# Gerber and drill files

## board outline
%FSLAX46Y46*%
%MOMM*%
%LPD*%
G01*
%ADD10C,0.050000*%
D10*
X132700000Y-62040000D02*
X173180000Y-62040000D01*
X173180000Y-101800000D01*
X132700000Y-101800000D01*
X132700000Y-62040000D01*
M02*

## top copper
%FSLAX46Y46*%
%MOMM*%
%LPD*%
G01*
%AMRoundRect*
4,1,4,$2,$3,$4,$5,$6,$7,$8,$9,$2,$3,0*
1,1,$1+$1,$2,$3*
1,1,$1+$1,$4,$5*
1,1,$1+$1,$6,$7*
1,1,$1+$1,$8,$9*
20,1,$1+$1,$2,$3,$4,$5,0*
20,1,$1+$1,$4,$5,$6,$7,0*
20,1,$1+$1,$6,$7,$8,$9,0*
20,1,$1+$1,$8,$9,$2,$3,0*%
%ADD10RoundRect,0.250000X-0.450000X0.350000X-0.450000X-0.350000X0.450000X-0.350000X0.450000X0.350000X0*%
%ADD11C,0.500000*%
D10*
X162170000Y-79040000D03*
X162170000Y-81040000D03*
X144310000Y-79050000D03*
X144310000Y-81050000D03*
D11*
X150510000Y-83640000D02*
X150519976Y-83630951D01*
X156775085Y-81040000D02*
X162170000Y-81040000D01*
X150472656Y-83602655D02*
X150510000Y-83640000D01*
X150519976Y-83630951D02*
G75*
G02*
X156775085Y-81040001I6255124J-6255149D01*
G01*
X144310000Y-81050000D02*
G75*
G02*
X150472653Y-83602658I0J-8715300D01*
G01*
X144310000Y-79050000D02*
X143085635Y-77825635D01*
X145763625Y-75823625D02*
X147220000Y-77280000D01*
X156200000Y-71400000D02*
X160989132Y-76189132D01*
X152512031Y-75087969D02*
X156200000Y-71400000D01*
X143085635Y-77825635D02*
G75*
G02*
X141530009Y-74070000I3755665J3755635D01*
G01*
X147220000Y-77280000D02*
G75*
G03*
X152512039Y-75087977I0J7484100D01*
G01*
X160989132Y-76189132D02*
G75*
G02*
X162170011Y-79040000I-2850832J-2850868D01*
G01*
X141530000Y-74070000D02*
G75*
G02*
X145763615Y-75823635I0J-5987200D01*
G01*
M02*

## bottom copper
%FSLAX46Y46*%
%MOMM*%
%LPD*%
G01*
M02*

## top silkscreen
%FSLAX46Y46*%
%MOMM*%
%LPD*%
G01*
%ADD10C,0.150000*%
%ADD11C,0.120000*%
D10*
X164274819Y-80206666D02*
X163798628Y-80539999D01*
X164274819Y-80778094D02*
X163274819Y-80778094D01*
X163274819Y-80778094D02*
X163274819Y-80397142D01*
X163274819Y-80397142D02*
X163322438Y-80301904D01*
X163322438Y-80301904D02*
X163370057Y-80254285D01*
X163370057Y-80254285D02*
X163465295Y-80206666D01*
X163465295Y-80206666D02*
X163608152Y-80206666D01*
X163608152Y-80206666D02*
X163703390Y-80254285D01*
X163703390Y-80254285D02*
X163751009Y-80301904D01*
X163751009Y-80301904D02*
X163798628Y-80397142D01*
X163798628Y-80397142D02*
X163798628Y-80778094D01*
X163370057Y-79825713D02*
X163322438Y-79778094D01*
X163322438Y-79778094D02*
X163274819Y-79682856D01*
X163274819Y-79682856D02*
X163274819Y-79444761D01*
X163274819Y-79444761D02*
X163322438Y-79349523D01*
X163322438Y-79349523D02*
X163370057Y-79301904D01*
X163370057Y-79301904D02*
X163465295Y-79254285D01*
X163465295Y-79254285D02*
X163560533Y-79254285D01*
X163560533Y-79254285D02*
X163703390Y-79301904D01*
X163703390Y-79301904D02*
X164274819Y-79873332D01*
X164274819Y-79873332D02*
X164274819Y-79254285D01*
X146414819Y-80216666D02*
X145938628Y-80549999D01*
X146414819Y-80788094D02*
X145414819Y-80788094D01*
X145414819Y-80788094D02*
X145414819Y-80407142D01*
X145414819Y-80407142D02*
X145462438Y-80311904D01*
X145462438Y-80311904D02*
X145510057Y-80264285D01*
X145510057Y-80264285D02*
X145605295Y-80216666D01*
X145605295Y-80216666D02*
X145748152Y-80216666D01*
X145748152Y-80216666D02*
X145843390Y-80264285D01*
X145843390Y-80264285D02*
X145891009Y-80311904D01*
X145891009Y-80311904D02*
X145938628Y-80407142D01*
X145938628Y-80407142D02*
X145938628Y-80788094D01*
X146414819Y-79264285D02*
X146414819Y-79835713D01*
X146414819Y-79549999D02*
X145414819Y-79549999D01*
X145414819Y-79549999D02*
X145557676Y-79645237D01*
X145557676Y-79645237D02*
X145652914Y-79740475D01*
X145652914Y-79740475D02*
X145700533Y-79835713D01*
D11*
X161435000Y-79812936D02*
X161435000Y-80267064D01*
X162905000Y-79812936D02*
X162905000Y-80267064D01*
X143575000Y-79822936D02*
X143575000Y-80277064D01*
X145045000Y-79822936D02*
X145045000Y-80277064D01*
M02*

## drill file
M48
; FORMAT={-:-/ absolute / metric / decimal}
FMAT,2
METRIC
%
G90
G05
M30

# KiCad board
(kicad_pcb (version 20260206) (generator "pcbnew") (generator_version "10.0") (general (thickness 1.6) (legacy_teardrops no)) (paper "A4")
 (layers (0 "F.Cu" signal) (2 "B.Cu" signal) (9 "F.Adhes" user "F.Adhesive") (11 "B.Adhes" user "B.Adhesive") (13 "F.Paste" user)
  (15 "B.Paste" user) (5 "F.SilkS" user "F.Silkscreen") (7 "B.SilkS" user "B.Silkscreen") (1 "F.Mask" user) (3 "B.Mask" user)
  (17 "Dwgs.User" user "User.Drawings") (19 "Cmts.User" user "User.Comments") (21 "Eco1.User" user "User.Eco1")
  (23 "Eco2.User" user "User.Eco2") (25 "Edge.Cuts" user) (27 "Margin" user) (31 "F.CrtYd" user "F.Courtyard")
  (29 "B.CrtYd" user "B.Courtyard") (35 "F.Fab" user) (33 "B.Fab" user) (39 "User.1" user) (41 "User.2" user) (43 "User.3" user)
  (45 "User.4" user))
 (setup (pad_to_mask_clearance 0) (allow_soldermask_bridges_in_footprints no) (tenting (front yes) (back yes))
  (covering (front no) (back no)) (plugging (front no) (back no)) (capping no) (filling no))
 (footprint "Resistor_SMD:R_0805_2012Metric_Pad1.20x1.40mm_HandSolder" (layer "F.Cu") (at 162.17 80.04 -90)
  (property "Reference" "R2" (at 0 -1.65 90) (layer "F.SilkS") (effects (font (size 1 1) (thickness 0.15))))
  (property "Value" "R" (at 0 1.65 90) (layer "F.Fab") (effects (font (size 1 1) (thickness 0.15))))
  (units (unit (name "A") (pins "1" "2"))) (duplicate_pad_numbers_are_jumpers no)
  (fp_line (start -0.227064 0.735) (end 0.227064 0.735) (stroke (width 0.12) (type solid)) (layer "F.SilkS"))
  (fp_line (start -0.227064 -0.735) (end 0.227064 -0.735) (stroke (width 0.12) (type solid)) (layer "F.SilkS"))
  (pad "1" smd roundrect (at -1 0 270) (size 1.2 1.4) (layers "F.Cu" "F.Mask" "F.Paste") (roundrect_rratio 0.208333) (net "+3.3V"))
  (pad "2" smd roundrect (at 1 0 270) (size 1.2 1.4) (layers "F.Cu" "F.Mask" "F.Paste") (roundrect_rratio 0.208333) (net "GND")))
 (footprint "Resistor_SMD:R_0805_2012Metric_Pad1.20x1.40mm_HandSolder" (layer "F.Cu") (at 144.31 80.05 -90)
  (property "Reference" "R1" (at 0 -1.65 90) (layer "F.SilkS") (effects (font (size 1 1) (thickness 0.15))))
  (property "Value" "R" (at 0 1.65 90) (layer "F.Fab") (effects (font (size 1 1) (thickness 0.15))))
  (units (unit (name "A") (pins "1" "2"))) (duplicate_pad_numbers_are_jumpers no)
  (fp_line (start -0.227064 0.735) (end 0.227064 0.735) (stroke (width 0.12) (type solid)) (layer "F.SilkS"))
  (fp_line (start -0.227064 -0.735) (end 0.227064 -0.735) (stroke (width 0.12) (type solid)) (layer "F.SilkS"))
  (pad "1" smd roundrect (at -1 0 270) (size 1.2 1.4) (layers "F.Cu" "F.Mask" "F.Paste") (roundrect_rratio 0.208333) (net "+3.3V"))
  (pad "2" smd roundrect (at 1 0 270) (size 1.2 1.4) (layers "F.Cu" "F.Mask" "F.Paste") (roundrect_rratio 0.208333) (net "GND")))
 (gr_rect (start 132.7 62.04) (end 173.18 101.8) (stroke (width 0.05) (type default)) (fill no) (layer "Edge.Cuts"))
 (segment (start 150.51 83.64) (end 150.519976 83.630951) (width 0.5) (layer "F.Cu") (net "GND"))
 (segment (start 156.775085 81.04) (end 162.17 81.04) (width 0.5) (layer "F.Cu") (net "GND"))
 (segment (start 150.472656 83.602655) (end 150.51 83.64) (width 0.5) (layer "F.Cu") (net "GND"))
 (arc (start 150.519976 83.630951) (mid 153.389844 81.713366) (end 156.775085 81.04) (width 0.5) (layer "F.Cu") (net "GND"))
 (arc (start 144.31 81.05) (mid 147.645205 81.713414) (end 150.472656 83.602655) (width 0.5) (layer "F.Cu") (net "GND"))
 (segment (start 144.31 79.05) (end 143.085635 77.825635) (width 0.5) (layer "F.Cu") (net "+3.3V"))
 (segment (start 145.763625 75.823625) (end 147.22 77.28) (width 0.5) (layer "F.Cu") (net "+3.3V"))
 (segment (start 156.2 71.4) (end 160.989132 76.189132) (width 0.5) (layer "F.Cu") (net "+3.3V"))
 (segment (start 152.512031 75.087969) (end 156.2 71.4) (width 0.5) (layer "F.Cu") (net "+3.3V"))
 (arc (start 143.085635 77.825635) (mid 141.934296 76.102535) (end 141.53 74.07) (width 0.5) (layer "F.Cu") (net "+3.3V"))
 (arc (start 147.22 77.28) (mid 150.084027 76.71031) (end 152.512031 75.087969) (width 0.5) (layer "F.Cu") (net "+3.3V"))
 (arc (start 160.989132 76.189132) (mid 161.863102 77.497122) (end 162.17 79.04) (width 0.5) (layer "F.Cu") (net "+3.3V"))
 (arc (start 141.53 74.07) (mid 143.821221 74.525752) (end 145.763625 75.823625) (width 0.5) (layer "F.Cu") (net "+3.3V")))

